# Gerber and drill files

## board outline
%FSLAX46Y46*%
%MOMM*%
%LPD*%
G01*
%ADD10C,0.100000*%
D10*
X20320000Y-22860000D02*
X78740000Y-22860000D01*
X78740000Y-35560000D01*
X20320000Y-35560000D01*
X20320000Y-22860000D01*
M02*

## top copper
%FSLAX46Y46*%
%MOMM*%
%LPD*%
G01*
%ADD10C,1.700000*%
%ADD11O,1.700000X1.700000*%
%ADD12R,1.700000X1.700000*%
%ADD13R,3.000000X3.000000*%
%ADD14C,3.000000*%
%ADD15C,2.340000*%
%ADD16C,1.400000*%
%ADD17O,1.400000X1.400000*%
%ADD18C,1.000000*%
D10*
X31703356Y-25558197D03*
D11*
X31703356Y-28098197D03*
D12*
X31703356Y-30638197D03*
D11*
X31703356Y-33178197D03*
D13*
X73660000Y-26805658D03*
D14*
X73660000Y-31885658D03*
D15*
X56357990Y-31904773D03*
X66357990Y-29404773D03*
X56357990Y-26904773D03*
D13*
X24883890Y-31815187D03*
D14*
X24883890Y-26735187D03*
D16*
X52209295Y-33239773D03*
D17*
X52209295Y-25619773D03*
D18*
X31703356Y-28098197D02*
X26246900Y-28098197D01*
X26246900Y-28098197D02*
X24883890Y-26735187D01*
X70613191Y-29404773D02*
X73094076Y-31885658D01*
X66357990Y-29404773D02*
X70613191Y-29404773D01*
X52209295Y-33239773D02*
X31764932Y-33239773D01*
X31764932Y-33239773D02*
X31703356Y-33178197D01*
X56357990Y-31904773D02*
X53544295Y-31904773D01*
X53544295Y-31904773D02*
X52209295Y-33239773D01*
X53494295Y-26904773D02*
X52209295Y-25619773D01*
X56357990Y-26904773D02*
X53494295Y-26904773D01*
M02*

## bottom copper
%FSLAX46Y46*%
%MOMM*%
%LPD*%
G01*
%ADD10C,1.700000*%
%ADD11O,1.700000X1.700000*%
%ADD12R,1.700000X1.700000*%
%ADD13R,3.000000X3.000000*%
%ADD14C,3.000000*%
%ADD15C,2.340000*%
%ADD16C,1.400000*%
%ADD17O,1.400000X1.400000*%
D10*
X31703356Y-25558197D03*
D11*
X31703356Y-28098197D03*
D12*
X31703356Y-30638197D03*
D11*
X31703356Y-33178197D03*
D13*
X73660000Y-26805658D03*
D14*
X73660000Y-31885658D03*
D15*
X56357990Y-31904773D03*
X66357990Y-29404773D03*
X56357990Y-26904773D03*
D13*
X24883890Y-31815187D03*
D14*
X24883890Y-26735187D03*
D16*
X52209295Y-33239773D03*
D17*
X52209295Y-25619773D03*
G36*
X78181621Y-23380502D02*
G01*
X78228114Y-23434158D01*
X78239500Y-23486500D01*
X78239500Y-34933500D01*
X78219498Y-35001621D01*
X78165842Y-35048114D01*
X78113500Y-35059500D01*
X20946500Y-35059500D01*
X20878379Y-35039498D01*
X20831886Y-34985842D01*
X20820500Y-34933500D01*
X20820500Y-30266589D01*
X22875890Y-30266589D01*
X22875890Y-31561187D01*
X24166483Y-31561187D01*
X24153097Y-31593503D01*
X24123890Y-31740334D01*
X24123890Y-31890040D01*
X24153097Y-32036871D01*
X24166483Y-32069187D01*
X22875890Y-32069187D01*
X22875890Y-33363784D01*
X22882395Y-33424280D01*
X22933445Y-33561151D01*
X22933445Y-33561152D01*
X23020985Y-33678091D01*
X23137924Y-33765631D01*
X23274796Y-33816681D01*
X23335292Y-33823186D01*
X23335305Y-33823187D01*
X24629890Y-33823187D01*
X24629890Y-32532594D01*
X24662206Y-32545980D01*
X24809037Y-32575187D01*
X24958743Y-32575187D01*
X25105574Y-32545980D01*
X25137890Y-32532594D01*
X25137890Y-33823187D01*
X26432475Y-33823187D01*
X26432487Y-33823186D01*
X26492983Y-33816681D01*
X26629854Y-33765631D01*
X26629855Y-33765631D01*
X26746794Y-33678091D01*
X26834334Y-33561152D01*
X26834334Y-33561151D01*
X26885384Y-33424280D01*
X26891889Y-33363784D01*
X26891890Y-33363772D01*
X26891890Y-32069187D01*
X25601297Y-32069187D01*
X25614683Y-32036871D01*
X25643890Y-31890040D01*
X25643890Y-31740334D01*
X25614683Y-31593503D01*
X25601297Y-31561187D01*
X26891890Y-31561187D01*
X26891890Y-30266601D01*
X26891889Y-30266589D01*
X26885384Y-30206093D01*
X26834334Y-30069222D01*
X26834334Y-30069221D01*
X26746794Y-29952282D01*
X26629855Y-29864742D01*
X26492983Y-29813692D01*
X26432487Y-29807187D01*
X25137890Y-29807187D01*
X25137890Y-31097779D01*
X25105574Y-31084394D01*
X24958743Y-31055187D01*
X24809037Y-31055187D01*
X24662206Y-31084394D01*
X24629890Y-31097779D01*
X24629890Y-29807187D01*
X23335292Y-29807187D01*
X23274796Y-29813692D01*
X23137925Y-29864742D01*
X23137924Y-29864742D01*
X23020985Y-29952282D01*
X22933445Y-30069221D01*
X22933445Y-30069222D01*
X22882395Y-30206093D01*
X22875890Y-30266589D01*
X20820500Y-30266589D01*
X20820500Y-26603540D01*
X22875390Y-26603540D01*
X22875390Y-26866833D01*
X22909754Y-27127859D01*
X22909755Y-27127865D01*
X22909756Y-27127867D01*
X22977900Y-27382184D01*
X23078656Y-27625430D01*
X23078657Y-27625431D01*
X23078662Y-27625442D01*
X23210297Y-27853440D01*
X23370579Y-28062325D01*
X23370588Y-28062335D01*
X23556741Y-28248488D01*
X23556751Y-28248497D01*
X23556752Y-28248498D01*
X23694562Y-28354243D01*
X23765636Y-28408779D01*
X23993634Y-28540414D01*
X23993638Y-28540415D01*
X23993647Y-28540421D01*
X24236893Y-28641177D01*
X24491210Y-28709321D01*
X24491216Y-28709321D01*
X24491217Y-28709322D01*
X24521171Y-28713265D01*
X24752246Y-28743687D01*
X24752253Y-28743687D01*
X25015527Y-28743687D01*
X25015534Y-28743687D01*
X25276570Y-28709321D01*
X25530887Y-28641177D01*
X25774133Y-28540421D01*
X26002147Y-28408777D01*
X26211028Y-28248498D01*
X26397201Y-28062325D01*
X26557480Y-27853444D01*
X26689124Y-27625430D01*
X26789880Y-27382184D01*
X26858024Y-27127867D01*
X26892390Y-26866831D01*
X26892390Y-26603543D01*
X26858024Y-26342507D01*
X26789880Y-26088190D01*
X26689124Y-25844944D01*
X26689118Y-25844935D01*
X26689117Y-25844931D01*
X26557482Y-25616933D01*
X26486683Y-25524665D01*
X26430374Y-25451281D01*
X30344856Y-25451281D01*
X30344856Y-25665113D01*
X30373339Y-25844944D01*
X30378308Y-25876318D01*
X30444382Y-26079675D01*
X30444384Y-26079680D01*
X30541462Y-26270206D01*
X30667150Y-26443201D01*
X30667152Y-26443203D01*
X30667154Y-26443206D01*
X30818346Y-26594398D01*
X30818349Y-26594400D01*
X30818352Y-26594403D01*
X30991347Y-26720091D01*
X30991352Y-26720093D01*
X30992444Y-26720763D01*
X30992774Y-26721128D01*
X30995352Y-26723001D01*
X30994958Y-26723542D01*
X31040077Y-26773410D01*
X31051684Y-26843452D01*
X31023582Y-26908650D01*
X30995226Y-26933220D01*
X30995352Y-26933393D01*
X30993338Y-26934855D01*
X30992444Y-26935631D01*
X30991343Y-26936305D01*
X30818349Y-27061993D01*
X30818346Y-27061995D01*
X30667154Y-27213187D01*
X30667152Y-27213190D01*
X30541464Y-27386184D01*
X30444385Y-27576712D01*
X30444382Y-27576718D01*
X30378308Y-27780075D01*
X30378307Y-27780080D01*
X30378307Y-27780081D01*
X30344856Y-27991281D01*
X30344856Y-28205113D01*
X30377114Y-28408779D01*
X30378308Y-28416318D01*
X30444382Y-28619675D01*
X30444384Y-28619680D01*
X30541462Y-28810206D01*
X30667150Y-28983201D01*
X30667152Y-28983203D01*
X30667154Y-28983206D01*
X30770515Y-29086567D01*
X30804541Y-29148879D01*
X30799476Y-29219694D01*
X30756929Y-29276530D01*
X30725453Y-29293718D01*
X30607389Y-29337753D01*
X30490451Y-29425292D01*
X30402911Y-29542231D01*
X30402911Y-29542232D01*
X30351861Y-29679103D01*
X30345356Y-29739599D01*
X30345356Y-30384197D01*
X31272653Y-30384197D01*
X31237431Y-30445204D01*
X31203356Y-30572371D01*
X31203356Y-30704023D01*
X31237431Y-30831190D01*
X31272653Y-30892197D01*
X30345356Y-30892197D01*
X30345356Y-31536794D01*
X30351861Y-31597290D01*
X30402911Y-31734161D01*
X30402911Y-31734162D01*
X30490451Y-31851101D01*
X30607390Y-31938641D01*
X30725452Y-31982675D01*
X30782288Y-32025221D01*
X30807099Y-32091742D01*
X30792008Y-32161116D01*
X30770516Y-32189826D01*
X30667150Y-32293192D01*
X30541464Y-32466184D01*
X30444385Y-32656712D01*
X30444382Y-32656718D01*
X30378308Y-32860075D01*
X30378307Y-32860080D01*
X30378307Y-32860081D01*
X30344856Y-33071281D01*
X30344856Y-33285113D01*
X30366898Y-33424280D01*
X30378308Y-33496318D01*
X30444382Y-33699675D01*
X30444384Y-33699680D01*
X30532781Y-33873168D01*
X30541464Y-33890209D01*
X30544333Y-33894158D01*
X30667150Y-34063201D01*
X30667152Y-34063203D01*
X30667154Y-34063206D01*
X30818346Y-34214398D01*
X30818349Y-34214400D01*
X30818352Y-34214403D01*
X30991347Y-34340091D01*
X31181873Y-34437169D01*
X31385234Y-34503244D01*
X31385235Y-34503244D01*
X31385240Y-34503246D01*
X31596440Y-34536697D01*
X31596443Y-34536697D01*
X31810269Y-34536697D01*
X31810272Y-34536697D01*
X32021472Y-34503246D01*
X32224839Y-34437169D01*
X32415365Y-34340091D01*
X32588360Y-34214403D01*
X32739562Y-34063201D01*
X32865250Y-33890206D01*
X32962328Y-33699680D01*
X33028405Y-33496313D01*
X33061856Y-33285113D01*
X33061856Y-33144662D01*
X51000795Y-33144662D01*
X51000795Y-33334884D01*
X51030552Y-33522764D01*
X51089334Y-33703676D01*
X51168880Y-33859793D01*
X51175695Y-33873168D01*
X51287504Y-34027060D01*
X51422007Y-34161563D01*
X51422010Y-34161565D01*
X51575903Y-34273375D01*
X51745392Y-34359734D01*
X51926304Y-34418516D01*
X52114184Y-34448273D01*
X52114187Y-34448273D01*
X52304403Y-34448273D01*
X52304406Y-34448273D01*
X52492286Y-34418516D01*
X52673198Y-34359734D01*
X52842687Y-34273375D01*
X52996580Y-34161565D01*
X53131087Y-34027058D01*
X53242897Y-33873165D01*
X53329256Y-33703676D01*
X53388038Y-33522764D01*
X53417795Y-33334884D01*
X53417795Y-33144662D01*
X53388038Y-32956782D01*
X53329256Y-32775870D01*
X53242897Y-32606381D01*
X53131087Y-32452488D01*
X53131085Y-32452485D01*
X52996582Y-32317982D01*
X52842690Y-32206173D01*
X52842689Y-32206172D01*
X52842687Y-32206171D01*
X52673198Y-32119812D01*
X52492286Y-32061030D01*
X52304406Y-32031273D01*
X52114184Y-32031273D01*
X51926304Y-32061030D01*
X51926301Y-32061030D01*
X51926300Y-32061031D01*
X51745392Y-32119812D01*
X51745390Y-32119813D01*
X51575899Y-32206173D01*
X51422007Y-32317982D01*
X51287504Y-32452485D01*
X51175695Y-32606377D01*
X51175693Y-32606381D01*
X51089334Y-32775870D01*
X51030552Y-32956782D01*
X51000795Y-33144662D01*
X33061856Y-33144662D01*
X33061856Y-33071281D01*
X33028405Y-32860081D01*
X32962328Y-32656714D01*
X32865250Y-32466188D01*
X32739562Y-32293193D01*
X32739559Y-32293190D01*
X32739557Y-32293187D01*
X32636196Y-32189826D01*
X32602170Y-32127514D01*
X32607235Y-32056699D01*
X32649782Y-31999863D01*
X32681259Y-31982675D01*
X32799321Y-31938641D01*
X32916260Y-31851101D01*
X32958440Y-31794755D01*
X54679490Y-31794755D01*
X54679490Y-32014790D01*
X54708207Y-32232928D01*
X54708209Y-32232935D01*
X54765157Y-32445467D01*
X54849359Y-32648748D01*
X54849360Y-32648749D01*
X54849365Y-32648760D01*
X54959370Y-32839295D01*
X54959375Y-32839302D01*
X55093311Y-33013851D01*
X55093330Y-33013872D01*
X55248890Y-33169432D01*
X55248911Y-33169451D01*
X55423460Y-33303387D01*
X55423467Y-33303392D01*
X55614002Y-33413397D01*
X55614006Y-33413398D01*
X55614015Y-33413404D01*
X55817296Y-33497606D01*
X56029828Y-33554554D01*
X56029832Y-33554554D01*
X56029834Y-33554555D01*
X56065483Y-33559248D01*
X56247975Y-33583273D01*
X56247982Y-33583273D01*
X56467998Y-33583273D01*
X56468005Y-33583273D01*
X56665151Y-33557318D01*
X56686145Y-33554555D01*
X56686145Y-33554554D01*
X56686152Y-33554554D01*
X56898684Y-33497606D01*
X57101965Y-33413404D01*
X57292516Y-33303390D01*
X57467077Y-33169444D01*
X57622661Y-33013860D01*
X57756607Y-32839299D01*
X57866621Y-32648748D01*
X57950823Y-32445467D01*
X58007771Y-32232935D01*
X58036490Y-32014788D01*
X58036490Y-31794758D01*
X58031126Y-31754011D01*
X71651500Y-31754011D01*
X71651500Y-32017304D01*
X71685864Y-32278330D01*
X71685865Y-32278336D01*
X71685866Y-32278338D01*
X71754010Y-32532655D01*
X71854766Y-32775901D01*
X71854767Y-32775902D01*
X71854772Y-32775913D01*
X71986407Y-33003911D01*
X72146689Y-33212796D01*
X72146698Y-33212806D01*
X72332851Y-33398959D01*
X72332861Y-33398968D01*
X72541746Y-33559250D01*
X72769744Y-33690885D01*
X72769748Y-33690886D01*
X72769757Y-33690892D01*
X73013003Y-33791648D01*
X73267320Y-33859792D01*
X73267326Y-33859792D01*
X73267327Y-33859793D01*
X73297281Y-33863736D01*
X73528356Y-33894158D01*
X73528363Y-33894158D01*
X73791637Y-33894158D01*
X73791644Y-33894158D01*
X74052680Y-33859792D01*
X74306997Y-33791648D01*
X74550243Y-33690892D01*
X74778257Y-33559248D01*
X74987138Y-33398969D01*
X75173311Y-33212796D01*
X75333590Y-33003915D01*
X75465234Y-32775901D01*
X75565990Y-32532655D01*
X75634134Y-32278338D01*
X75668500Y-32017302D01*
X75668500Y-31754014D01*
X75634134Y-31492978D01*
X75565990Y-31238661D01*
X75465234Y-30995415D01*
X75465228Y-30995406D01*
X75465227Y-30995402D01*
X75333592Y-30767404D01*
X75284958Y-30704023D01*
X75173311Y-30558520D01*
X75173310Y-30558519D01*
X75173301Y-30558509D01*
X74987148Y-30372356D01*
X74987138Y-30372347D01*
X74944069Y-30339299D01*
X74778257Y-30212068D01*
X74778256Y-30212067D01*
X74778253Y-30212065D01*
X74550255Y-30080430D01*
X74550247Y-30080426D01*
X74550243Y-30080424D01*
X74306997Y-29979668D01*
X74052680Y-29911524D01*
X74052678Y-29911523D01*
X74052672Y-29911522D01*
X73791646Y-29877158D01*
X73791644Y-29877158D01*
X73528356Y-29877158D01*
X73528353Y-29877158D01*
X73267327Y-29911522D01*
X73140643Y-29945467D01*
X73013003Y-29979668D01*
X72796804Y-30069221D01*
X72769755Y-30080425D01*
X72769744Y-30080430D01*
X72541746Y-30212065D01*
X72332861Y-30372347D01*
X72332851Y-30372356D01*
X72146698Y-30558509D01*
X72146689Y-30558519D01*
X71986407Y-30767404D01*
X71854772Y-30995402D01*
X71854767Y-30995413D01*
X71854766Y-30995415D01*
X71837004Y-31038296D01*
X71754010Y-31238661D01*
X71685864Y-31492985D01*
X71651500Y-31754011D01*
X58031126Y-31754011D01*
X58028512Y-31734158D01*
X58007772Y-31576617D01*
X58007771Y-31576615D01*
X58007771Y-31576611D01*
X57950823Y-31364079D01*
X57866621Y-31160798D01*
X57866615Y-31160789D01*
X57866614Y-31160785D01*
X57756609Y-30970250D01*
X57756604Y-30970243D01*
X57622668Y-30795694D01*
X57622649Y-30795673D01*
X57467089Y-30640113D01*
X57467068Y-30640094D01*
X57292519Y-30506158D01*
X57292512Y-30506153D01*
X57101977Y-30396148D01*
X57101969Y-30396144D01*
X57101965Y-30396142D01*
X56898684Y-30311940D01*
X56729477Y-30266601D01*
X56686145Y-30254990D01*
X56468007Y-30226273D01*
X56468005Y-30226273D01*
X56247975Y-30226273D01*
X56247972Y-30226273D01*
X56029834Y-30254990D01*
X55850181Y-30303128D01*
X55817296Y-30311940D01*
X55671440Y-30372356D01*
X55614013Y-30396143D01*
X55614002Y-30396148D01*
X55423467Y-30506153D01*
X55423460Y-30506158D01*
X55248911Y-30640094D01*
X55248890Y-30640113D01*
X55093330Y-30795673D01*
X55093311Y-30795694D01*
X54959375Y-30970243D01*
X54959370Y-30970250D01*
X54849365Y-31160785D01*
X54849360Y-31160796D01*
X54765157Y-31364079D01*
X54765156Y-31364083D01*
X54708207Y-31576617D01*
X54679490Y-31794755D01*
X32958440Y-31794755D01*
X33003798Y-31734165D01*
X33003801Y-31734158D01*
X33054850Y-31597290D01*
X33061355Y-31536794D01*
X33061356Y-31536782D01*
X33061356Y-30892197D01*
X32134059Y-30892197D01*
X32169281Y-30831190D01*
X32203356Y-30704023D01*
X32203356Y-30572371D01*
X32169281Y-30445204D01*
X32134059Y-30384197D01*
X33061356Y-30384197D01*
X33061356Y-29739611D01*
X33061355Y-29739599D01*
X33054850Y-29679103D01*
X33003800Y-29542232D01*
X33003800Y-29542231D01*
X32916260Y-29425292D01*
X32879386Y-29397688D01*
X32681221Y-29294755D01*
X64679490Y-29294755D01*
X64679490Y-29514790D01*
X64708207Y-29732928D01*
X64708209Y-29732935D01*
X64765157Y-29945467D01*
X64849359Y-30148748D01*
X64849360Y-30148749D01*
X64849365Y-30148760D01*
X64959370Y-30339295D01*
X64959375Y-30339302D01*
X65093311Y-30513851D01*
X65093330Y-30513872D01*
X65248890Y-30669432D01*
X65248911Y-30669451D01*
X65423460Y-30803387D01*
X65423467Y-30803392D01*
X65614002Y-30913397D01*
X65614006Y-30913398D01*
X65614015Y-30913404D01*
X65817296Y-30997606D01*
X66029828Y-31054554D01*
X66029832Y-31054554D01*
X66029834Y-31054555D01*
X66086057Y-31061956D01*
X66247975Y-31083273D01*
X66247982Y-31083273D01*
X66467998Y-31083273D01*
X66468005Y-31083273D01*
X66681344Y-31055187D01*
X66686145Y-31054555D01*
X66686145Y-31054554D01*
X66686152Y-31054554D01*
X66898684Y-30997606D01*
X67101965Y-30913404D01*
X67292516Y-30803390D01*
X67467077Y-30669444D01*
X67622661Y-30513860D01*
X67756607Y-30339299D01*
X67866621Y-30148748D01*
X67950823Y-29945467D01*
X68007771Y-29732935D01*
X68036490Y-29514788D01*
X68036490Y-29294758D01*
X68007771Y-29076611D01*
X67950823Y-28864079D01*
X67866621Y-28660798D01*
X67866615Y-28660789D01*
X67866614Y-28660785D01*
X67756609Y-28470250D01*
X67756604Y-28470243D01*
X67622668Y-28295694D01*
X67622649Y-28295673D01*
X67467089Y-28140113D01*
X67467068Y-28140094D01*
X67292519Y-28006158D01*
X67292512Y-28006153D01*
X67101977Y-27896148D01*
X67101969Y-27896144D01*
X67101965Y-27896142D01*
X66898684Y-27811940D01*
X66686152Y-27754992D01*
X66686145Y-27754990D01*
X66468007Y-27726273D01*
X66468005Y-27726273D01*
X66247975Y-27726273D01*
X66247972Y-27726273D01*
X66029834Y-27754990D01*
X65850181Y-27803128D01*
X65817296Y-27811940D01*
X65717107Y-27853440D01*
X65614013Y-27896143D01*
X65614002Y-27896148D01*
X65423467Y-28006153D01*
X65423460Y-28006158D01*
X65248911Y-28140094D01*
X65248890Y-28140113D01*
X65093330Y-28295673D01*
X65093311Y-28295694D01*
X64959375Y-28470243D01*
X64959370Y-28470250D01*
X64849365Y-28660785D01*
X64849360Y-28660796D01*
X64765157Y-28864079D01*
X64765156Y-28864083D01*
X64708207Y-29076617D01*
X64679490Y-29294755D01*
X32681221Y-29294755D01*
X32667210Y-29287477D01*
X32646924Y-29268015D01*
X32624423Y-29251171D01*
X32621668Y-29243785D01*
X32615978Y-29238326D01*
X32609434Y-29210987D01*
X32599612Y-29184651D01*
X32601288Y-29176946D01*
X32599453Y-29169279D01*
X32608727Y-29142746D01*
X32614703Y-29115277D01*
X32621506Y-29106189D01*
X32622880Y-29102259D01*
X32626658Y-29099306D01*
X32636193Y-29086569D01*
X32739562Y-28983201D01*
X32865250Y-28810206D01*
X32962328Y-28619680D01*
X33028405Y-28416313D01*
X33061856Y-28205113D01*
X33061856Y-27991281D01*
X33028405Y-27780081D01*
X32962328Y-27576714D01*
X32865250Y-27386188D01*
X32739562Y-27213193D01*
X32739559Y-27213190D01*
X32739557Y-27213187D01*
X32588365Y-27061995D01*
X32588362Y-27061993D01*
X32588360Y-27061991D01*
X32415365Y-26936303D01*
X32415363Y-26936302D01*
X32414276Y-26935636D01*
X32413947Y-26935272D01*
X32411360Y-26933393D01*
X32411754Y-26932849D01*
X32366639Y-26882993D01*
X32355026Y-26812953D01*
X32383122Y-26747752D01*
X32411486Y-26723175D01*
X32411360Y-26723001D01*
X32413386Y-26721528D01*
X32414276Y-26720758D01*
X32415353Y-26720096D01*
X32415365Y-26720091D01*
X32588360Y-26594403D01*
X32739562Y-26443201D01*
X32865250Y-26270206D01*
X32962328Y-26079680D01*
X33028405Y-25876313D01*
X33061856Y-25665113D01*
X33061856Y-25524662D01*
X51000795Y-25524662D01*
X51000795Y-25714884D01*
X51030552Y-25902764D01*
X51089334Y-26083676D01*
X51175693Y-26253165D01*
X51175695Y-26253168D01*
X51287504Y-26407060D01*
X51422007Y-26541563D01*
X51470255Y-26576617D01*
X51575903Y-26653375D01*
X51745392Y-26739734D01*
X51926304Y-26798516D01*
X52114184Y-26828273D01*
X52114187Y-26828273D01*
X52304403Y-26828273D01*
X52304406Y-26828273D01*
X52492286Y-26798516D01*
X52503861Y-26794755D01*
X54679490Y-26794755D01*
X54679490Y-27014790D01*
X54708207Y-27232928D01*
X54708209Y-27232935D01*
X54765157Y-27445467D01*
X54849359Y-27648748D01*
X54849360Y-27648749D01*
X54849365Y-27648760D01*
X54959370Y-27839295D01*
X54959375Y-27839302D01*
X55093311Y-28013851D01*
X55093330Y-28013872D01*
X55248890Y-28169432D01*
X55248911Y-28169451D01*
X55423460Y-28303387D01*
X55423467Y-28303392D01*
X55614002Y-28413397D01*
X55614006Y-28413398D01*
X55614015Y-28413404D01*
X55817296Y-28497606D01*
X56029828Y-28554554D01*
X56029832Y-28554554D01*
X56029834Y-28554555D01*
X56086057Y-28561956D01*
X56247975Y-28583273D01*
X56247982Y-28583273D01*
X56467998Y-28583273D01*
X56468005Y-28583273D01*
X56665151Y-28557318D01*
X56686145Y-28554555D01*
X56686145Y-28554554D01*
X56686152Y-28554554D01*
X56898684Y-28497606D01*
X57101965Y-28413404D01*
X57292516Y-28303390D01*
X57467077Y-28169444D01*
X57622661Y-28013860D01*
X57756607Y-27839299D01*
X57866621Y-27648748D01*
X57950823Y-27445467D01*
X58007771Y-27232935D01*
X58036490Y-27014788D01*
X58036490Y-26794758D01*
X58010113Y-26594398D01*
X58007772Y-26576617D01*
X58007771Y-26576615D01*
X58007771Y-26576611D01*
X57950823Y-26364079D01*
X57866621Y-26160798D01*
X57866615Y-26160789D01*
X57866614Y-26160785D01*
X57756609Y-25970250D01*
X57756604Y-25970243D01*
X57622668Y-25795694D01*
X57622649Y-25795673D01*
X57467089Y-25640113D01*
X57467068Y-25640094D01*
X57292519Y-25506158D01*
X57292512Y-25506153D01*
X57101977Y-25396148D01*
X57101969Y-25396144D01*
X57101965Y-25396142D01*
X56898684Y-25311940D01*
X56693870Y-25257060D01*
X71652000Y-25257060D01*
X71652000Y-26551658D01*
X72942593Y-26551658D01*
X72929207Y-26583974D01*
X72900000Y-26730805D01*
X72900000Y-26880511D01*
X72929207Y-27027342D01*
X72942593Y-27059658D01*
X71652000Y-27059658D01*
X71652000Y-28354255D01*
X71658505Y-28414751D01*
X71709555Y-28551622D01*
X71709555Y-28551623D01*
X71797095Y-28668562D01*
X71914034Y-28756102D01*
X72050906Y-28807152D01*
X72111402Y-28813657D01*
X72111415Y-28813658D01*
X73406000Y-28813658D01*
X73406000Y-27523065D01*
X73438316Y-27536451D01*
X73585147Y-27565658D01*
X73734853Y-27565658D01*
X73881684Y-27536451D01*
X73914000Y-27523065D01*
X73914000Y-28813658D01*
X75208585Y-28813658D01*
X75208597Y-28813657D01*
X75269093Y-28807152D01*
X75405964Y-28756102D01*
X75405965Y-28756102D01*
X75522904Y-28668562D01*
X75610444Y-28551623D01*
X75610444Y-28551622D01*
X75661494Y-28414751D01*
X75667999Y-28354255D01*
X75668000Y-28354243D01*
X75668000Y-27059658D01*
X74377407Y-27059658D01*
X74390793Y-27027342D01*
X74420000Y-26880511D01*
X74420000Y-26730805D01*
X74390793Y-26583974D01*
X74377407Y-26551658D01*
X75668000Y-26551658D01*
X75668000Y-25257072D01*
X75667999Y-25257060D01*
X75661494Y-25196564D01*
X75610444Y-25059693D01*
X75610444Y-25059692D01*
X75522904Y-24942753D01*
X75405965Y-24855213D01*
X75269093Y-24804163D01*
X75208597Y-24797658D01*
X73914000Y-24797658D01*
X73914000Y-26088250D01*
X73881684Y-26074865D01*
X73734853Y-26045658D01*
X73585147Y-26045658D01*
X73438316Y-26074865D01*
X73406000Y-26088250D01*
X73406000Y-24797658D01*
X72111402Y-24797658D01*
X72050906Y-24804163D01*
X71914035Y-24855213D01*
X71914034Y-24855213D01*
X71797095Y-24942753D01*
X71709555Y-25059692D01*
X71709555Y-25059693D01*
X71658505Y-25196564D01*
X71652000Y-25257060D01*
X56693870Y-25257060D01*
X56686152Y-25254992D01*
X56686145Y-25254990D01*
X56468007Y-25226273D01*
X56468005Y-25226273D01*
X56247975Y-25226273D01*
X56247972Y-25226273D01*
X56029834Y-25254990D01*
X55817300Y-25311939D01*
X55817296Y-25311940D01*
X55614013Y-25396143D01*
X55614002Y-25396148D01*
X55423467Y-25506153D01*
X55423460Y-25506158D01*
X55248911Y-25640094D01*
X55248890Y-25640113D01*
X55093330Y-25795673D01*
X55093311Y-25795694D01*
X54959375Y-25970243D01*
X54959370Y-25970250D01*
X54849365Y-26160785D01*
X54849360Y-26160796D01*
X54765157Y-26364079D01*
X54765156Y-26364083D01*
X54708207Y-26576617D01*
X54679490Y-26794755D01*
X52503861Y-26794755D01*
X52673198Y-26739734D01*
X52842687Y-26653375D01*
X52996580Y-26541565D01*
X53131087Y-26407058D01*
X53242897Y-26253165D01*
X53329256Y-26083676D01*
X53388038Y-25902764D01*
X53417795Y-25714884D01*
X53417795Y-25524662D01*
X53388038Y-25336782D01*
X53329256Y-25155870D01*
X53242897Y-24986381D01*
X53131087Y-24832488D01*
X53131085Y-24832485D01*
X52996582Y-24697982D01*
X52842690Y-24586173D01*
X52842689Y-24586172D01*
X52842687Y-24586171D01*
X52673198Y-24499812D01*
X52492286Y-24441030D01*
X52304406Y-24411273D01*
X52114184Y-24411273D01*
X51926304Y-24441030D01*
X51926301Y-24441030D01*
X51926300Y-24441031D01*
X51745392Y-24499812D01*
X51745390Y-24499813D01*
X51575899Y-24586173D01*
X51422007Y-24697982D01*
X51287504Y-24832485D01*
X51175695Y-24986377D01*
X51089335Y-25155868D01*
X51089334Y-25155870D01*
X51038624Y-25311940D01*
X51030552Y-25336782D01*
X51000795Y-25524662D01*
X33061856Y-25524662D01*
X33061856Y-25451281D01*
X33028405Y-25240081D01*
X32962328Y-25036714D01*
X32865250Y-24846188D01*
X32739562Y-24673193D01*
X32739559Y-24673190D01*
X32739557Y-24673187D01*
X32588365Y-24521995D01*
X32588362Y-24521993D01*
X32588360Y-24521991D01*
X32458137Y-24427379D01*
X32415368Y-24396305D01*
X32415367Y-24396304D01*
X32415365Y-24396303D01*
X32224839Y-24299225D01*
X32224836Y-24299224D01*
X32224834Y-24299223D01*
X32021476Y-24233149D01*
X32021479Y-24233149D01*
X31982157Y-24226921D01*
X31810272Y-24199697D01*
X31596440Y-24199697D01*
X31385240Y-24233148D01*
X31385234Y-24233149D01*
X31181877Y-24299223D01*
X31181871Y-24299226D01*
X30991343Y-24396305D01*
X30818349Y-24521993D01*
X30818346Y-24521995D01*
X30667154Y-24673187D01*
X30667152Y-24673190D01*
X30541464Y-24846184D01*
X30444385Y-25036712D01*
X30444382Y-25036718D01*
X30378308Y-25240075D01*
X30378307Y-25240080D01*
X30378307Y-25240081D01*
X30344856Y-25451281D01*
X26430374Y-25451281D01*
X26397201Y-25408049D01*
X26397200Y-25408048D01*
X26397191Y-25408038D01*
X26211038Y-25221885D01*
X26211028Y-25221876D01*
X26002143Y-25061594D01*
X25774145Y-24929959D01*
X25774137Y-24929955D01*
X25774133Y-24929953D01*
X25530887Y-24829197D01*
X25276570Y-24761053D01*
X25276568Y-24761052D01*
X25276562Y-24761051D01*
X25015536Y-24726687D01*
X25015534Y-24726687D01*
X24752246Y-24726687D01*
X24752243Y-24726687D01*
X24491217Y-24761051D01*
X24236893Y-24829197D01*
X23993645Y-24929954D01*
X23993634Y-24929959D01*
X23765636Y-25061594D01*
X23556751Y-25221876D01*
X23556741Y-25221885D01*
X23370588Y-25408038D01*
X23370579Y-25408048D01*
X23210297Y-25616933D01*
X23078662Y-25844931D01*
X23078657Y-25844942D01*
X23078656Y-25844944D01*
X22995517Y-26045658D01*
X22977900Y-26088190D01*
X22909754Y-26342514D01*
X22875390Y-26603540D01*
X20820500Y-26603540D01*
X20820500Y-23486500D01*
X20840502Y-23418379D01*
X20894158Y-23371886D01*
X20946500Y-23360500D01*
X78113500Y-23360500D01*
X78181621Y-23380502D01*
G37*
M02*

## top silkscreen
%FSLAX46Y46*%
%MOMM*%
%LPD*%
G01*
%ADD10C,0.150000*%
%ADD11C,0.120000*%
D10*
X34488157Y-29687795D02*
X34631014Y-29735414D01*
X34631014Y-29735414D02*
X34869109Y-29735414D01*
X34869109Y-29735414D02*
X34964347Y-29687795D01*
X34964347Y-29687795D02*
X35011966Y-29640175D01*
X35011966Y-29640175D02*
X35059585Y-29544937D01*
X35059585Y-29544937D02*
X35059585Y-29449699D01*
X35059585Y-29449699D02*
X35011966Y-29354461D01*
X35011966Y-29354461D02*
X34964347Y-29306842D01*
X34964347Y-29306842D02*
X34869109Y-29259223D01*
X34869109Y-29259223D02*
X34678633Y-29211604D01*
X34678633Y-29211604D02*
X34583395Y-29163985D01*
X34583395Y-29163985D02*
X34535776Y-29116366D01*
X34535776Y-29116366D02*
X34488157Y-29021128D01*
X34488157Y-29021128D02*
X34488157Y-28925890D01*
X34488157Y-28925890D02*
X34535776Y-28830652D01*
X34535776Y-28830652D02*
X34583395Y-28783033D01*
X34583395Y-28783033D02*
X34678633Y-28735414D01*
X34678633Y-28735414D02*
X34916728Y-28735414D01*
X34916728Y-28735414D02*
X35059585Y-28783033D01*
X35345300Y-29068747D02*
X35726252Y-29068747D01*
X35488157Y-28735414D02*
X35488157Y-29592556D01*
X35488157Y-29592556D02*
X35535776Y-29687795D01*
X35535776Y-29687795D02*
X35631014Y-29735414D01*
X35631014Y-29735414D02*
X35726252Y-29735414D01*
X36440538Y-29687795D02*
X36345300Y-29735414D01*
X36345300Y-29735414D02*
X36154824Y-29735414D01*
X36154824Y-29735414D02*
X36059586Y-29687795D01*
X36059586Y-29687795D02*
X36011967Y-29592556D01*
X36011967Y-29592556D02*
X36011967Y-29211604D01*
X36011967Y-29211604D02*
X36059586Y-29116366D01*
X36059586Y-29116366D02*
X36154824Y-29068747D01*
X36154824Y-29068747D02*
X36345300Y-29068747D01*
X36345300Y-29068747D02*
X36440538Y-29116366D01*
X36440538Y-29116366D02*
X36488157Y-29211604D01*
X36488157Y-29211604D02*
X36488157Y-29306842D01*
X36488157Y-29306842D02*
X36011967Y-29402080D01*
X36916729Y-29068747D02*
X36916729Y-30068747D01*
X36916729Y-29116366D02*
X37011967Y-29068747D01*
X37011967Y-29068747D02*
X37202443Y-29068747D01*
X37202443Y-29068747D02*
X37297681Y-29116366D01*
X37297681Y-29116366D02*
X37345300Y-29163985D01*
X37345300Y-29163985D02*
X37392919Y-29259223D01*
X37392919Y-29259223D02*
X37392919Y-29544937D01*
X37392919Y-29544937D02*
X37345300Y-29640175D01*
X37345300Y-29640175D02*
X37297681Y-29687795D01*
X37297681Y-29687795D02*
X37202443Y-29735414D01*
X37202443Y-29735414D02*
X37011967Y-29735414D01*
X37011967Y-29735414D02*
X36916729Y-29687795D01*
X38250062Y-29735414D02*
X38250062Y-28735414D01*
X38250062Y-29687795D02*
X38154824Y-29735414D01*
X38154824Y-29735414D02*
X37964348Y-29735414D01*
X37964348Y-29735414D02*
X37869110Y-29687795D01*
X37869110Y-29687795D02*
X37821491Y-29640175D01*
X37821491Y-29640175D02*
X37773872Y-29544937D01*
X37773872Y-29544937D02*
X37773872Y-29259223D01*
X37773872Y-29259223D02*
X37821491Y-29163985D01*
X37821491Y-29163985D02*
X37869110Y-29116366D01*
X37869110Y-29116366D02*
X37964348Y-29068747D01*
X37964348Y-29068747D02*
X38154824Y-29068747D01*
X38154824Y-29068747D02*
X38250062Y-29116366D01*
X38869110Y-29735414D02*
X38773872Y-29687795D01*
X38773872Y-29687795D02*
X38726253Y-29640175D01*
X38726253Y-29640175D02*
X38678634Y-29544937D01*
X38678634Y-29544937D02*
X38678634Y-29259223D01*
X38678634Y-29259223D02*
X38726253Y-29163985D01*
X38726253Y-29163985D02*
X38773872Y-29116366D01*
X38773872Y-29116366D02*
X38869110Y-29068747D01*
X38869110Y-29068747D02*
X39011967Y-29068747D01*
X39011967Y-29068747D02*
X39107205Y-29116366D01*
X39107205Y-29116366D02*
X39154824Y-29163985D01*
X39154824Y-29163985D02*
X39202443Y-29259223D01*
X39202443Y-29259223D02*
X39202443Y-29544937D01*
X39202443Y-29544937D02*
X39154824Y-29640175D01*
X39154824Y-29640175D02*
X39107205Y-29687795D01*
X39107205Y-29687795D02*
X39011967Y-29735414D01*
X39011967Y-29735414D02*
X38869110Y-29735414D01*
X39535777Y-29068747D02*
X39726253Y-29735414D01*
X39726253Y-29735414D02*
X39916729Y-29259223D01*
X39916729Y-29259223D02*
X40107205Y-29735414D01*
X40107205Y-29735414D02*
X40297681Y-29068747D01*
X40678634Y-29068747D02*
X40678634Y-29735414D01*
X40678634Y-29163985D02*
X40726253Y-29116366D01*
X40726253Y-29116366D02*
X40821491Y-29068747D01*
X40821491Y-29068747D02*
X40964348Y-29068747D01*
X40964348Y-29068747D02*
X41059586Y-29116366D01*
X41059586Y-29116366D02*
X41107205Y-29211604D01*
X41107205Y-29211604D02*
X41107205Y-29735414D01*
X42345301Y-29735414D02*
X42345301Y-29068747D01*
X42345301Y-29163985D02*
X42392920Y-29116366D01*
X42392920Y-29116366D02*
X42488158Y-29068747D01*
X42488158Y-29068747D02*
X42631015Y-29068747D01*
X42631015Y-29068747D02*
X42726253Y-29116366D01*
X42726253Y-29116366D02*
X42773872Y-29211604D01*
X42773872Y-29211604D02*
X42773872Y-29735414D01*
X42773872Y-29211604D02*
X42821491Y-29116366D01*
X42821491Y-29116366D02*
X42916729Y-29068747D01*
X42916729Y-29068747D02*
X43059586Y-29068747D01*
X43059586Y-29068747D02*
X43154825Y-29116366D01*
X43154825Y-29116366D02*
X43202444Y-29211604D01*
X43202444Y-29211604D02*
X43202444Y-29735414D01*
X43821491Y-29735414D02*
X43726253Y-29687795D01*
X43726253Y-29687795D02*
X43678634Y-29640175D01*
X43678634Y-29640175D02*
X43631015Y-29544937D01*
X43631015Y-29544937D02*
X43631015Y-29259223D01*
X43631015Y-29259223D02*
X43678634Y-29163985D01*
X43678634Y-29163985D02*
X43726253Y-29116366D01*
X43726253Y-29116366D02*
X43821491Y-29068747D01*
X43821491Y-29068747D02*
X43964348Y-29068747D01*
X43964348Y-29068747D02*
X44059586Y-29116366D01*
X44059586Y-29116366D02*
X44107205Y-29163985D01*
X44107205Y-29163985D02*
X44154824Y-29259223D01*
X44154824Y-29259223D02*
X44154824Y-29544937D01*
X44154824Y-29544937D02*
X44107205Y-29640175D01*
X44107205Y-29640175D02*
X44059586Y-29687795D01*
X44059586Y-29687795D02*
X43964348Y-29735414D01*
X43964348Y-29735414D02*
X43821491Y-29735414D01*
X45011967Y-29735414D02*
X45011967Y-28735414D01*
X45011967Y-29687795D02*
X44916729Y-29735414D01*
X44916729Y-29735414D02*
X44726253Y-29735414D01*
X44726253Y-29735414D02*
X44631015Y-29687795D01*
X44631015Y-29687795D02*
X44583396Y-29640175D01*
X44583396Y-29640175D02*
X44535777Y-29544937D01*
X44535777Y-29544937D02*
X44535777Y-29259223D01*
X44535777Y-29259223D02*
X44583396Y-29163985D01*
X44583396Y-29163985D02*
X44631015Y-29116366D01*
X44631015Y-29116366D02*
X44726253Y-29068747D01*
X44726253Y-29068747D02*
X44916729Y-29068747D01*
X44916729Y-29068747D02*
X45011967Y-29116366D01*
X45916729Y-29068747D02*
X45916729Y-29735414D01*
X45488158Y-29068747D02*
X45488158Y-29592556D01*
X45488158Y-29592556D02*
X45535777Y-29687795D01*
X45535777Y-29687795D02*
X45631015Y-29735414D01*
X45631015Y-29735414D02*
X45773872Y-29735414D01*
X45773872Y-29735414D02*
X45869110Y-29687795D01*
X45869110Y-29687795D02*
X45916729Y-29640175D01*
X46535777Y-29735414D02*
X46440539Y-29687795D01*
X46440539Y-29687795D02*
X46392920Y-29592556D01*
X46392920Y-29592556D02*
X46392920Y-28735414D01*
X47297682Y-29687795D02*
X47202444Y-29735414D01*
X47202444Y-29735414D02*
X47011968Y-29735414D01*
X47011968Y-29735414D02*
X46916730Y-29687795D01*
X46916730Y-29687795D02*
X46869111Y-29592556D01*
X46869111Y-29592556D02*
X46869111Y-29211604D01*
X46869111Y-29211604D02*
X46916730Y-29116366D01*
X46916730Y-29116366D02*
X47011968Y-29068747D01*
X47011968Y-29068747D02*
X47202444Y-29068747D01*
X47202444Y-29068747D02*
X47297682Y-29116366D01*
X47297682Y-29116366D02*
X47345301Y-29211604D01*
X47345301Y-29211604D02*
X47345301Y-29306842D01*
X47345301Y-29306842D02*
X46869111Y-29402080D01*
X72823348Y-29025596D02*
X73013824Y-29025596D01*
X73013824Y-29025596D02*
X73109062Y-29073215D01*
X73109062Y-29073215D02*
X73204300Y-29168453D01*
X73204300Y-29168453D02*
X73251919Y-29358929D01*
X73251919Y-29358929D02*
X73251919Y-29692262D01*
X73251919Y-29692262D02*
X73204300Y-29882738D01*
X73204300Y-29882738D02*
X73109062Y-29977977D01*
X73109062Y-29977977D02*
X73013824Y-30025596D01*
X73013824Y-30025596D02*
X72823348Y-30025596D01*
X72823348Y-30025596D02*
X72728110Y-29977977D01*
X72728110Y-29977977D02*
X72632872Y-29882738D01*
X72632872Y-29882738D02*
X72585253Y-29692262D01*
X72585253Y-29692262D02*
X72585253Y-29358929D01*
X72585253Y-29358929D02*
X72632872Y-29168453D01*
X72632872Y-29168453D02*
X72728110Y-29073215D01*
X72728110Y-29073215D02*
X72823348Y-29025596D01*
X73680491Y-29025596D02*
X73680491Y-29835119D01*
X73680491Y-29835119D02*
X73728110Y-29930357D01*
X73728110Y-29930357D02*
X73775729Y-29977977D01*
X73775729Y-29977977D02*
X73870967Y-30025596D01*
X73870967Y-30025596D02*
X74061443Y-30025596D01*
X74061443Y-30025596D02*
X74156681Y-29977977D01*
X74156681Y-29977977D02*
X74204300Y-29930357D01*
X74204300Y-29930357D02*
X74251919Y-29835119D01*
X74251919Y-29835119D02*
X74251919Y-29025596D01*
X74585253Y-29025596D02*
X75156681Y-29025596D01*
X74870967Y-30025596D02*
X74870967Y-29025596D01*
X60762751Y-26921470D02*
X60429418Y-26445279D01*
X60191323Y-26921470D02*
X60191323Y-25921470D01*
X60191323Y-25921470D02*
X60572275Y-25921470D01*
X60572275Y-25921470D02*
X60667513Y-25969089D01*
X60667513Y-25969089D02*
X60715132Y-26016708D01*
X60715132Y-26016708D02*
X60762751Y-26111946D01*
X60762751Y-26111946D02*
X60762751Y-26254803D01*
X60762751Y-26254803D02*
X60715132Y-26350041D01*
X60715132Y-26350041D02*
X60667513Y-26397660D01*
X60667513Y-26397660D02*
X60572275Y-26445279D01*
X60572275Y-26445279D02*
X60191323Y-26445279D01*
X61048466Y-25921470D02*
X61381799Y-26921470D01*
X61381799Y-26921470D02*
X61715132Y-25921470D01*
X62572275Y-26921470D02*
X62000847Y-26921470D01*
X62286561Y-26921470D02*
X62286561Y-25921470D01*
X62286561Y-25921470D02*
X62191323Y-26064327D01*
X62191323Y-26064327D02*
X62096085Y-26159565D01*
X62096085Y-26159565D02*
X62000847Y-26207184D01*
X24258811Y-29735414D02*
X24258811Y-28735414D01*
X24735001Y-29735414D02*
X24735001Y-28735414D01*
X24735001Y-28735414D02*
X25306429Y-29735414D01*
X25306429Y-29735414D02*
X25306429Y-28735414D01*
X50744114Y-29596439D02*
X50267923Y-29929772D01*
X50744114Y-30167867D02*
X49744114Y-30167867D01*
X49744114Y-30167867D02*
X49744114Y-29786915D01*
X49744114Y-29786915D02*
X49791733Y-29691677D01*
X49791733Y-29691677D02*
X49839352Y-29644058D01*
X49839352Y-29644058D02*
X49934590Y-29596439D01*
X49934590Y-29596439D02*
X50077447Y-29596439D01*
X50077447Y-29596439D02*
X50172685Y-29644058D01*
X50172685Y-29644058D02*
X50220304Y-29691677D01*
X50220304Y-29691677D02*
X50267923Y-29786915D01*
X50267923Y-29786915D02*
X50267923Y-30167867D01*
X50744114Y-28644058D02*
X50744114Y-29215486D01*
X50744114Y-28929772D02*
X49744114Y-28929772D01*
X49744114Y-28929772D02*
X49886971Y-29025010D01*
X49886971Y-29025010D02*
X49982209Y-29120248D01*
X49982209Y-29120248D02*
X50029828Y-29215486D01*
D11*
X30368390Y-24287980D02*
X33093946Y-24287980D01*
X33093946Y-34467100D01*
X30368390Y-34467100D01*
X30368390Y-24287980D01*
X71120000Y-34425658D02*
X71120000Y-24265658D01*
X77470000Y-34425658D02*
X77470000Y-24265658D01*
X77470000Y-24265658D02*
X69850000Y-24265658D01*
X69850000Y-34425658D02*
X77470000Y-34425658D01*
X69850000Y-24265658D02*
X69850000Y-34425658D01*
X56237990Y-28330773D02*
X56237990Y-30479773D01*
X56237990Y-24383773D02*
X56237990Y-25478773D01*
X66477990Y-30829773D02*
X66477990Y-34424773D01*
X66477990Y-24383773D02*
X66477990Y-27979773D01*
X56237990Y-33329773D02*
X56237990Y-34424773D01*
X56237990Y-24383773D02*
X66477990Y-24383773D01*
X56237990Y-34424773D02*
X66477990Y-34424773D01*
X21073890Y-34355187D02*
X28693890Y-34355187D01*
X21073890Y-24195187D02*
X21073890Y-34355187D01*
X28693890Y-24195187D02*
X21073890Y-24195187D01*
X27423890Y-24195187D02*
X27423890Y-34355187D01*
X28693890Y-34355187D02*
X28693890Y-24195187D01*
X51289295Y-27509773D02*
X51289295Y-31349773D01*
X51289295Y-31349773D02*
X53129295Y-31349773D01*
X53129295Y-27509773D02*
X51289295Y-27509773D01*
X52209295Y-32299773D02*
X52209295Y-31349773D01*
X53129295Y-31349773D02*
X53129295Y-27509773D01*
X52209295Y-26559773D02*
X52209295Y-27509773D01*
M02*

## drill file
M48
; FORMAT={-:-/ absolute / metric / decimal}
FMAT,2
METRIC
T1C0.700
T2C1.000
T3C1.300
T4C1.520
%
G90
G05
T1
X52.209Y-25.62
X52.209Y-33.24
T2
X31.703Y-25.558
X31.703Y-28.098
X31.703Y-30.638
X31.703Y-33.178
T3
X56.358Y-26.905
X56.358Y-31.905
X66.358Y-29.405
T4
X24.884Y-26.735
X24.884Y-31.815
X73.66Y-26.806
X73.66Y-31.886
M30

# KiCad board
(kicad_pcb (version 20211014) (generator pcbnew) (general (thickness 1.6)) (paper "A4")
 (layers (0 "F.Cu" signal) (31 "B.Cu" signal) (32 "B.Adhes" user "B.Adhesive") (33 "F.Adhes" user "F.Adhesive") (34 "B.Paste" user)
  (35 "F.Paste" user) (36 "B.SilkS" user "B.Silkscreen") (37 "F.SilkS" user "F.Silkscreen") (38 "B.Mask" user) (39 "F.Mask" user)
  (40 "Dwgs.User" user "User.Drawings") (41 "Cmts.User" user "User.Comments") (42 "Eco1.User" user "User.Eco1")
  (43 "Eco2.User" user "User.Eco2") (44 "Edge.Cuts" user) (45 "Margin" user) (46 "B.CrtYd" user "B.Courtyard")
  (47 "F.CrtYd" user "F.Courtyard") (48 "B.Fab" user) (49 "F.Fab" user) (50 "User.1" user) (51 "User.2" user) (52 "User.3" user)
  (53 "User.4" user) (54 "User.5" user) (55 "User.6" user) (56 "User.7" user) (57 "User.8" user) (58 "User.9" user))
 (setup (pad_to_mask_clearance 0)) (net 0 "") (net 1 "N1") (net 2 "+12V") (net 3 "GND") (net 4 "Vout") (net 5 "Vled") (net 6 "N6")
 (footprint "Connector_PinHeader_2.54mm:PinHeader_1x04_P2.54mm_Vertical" (layer "F.Cu") (at 31.703356 25.558197)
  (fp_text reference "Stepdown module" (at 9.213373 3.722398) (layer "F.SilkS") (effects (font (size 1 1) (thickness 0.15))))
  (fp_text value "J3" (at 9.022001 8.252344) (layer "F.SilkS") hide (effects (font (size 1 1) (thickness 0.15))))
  (fp_rect (start -1.334966 -1.270217) (end 1.39059 8.908903) (layer "F.SilkS") (width 0.12) (fill none))
  (pad "1" thru_hole circle (at 0 0) (size 1.7 1.7) (drill 1) (layers *.Cu *.Mask) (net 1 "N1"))
  (pad "2" thru_hole oval (at 0 2.54) (size 1.7 1.7) (drill 1) (layers *.Cu *.Mask) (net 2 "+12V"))
  (pad "3" thru_hole rect (at 0 5.08) (size 1.7 1.7) (drill 1) (layers *.Cu *.Mask) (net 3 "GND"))
  (pad "4" thru_hole oval (at 0 7.62) (size 1.7 1.7) (drill 1) (layers *.Cu *.Mask) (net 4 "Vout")))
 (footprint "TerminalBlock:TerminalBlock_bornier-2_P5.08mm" (layer "F.Cu") (at 73.66 26.805658 -90)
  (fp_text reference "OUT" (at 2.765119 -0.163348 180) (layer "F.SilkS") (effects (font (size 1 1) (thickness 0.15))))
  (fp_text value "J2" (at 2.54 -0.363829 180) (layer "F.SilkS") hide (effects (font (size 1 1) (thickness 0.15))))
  (fp_line (start 7.62 2.54) (end -2.54 2.54) (layer "F.SilkS") (width 0.12))
  (fp_line (start 7.62 -3.81) (end -2.54 -3.81) (layer "F.SilkS") (width 0.12))
  (fp_line (start -2.54 -3.81) (end -2.54 3.81) (layer "F.SilkS") (width 0.12))
  (fp_line (start 7.62 3.81) (end 7.62 -3.81) (layer "F.SilkS") (width 0.12))
  (fp_line (start -2.54 3.81) (end 7.62 3.81) (layer "F.SilkS") (width 0.12))
  (pad "1" thru_hole rect (at 0 0 270) (size 3 3) (drill 1.52) (layers *.Cu *.Mask) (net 3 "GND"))
  (pad "2" thru_hole circle (at 5.08 0 270) (size 3 3) (drill 1.52) (layers *.Cu *.Mask) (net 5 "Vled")))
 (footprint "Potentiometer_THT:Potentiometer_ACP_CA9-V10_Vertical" (layer "F.Cu") (at 56.35799 31.904773)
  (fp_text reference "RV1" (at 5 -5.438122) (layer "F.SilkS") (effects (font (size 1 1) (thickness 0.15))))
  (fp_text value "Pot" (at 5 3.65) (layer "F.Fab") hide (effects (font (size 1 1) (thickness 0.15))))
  (fp_line (start -0.12 -3.574) (end -0.12 -1.425) (layer "F.SilkS") (width 0.12))
  (fp_line (start -0.12 -7.521) (end -0.12 -6.426) (layer "F.SilkS") (width 0.12))
  (fp_line (start 10.12 -1.075) (end 10.12 2.52) (layer "F.SilkS") (width 0.12))
  (fp_line (start 10.12 -7.521) (end 10.12 -3.925) (layer "F.SilkS") (width 0.12))
  (fp_line (start -0.12 1.425) (end -0.12 2.52) (layer "F.SilkS") (width 0.12))
  (fp_line (start -0.12 -7.521) (end 10.12 -7.521) (layer "F.SilkS") (width 0.12))
  (fp_line (start -0.12 2.52) (end 10.12 2.52) (layer "F.SilkS") (width 0.12))
  (pad "1" thru_hole circle (at 0 0) (size 2.34 2.34) (drill 1.3) (layers *.Cu *.Mask) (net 4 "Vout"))
  (pad "2" thru_hole circle (at 10 -2.5) (size 2.34 2.34) (drill 1.3) (layers *.Cu *.Mask) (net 5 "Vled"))
  (pad "3" thru_hole circle (at 0 -5) (size 2.34 2.34) (drill 1.3) (layers *.Cu *.Mask) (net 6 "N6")))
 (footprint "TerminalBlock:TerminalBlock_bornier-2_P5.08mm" (layer "F.Cu") (at 24.88389 31.815187 90)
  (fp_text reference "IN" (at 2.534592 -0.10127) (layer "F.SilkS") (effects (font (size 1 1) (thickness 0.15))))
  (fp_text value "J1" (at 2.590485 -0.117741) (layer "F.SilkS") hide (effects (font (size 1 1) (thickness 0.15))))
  (fp_line (start -2.54 -3.81) (end -2.54 3.81) (layer "F.SilkS") (width 0.12))
  (fp_line (start 7.62 -3.81) (end -2.54 -3.81) (layer "F.SilkS") (width 0.12))
  (fp_line (start 7.62 3.81) (end 7.62 -3.81) (layer "F.SilkS") (width 0.12))
  (fp_line (start 7.62 2.54) (end -2.54 2.54) (layer "F.SilkS") (width 0.12))
  (fp_line (start -2.54 3.81) (end 7.62 3.81) (layer "F.SilkS") (width 0.12))
  (pad "1" thru_hole rect (at 0 0 90) (size 3 3) (drill 1.52) (layers *.Cu *.Mask) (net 3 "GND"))
  (pad "2" thru_hole circle (at 5.08 0 90) (size 3 3) (drill 1.52) (layers *.Cu *.Mask) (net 2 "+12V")))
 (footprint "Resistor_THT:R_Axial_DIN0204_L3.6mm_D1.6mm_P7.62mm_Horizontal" (layer "F.Cu") (at 52.209295 33.239773 90)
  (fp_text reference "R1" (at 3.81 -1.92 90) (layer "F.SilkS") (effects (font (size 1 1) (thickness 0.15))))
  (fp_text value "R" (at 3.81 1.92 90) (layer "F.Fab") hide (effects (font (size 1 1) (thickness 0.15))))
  (fp_line (start 5.73 -0.92) (end 1.89 -0.92) (layer "F.SilkS") (width 0.12))
  (fp_line (start 1.89 -0.92) (end 1.89 0.92) (layer "F.SilkS") (width 0.12))
  (fp_line (start 5.73 0.92) (end 5.73 -0.92) (layer "F.SilkS") (width 0.12))
  (fp_line (start 0.94 0) (end 1.89 0) (layer "F.SilkS") (width 0.12))
  (fp_line (start 1.89 0.92) (end 5.73 0.92) (layer "F.SilkS") (width 0.12))
  (fp_line (start 6.68 0) (end 5.73 0) (layer "F.SilkS") (width 0.12))
  (pad "1" thru_hole circle (at 0 0 90) (size 1.4 1.4) (drill 0.7) (layers *.Cu *.Mask) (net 4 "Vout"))
  (pad "2" thru_hole oval (at 7.62 0 90) (size 1.4 1.4) (drill 0.7) (layers *.Cu *.Mask) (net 6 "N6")))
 (gr_rect (start 20.32 22.86) (end 78.74 35.56) (layer "Edge.Cuts") (width 0.1) (fill none))
 (segment (start 31.703356 28.098197) (end 26.2469 28.098197) (width 1) (layer "F.Cu") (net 2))
 (segment (start 26.2469 28.098197) (end 24.88389 26.735187) (width 1) (layer "F.Cu") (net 2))
 (segment (start 70.613191 29.404773) (end 73.094076 31.885658) (width 1) (layer "F.Cu") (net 5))
 (segment (start 66.35799 29.404773) (end 70.613191 29.404773) (width 1) (layer "F.Cu") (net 5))
 (segment (start 52.209295 33.239773) (end 31.764932 33.239773) (width 1) (layer "F.Cu") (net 4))
 (segment (start 31.764932 33.239773) (end 31.703356 33.178197) (width 1) (layer "F.Cu") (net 4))
 (segment (start 56.35799 31.904773) (end 53.544295 31.904773) (width 1) (layer "F.Cu") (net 4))
 (segment (start 53.544295 31.904773) (end 52.209295 33.239773) (width 1) (layer "F.Cu") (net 4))
 (segment (start 53.494295 26.904773) (end 52.209295 25.619773) (width 1) (layer "F.Cu") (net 6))
 (segment (start 56.35799 26.904773) (end 53.494295 26.904773) (width 1) (layer "F.Cu") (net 6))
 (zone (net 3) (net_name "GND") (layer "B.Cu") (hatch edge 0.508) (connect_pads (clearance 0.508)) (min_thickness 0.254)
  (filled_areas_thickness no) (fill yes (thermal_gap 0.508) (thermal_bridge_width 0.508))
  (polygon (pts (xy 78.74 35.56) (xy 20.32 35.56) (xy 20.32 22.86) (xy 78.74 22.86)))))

